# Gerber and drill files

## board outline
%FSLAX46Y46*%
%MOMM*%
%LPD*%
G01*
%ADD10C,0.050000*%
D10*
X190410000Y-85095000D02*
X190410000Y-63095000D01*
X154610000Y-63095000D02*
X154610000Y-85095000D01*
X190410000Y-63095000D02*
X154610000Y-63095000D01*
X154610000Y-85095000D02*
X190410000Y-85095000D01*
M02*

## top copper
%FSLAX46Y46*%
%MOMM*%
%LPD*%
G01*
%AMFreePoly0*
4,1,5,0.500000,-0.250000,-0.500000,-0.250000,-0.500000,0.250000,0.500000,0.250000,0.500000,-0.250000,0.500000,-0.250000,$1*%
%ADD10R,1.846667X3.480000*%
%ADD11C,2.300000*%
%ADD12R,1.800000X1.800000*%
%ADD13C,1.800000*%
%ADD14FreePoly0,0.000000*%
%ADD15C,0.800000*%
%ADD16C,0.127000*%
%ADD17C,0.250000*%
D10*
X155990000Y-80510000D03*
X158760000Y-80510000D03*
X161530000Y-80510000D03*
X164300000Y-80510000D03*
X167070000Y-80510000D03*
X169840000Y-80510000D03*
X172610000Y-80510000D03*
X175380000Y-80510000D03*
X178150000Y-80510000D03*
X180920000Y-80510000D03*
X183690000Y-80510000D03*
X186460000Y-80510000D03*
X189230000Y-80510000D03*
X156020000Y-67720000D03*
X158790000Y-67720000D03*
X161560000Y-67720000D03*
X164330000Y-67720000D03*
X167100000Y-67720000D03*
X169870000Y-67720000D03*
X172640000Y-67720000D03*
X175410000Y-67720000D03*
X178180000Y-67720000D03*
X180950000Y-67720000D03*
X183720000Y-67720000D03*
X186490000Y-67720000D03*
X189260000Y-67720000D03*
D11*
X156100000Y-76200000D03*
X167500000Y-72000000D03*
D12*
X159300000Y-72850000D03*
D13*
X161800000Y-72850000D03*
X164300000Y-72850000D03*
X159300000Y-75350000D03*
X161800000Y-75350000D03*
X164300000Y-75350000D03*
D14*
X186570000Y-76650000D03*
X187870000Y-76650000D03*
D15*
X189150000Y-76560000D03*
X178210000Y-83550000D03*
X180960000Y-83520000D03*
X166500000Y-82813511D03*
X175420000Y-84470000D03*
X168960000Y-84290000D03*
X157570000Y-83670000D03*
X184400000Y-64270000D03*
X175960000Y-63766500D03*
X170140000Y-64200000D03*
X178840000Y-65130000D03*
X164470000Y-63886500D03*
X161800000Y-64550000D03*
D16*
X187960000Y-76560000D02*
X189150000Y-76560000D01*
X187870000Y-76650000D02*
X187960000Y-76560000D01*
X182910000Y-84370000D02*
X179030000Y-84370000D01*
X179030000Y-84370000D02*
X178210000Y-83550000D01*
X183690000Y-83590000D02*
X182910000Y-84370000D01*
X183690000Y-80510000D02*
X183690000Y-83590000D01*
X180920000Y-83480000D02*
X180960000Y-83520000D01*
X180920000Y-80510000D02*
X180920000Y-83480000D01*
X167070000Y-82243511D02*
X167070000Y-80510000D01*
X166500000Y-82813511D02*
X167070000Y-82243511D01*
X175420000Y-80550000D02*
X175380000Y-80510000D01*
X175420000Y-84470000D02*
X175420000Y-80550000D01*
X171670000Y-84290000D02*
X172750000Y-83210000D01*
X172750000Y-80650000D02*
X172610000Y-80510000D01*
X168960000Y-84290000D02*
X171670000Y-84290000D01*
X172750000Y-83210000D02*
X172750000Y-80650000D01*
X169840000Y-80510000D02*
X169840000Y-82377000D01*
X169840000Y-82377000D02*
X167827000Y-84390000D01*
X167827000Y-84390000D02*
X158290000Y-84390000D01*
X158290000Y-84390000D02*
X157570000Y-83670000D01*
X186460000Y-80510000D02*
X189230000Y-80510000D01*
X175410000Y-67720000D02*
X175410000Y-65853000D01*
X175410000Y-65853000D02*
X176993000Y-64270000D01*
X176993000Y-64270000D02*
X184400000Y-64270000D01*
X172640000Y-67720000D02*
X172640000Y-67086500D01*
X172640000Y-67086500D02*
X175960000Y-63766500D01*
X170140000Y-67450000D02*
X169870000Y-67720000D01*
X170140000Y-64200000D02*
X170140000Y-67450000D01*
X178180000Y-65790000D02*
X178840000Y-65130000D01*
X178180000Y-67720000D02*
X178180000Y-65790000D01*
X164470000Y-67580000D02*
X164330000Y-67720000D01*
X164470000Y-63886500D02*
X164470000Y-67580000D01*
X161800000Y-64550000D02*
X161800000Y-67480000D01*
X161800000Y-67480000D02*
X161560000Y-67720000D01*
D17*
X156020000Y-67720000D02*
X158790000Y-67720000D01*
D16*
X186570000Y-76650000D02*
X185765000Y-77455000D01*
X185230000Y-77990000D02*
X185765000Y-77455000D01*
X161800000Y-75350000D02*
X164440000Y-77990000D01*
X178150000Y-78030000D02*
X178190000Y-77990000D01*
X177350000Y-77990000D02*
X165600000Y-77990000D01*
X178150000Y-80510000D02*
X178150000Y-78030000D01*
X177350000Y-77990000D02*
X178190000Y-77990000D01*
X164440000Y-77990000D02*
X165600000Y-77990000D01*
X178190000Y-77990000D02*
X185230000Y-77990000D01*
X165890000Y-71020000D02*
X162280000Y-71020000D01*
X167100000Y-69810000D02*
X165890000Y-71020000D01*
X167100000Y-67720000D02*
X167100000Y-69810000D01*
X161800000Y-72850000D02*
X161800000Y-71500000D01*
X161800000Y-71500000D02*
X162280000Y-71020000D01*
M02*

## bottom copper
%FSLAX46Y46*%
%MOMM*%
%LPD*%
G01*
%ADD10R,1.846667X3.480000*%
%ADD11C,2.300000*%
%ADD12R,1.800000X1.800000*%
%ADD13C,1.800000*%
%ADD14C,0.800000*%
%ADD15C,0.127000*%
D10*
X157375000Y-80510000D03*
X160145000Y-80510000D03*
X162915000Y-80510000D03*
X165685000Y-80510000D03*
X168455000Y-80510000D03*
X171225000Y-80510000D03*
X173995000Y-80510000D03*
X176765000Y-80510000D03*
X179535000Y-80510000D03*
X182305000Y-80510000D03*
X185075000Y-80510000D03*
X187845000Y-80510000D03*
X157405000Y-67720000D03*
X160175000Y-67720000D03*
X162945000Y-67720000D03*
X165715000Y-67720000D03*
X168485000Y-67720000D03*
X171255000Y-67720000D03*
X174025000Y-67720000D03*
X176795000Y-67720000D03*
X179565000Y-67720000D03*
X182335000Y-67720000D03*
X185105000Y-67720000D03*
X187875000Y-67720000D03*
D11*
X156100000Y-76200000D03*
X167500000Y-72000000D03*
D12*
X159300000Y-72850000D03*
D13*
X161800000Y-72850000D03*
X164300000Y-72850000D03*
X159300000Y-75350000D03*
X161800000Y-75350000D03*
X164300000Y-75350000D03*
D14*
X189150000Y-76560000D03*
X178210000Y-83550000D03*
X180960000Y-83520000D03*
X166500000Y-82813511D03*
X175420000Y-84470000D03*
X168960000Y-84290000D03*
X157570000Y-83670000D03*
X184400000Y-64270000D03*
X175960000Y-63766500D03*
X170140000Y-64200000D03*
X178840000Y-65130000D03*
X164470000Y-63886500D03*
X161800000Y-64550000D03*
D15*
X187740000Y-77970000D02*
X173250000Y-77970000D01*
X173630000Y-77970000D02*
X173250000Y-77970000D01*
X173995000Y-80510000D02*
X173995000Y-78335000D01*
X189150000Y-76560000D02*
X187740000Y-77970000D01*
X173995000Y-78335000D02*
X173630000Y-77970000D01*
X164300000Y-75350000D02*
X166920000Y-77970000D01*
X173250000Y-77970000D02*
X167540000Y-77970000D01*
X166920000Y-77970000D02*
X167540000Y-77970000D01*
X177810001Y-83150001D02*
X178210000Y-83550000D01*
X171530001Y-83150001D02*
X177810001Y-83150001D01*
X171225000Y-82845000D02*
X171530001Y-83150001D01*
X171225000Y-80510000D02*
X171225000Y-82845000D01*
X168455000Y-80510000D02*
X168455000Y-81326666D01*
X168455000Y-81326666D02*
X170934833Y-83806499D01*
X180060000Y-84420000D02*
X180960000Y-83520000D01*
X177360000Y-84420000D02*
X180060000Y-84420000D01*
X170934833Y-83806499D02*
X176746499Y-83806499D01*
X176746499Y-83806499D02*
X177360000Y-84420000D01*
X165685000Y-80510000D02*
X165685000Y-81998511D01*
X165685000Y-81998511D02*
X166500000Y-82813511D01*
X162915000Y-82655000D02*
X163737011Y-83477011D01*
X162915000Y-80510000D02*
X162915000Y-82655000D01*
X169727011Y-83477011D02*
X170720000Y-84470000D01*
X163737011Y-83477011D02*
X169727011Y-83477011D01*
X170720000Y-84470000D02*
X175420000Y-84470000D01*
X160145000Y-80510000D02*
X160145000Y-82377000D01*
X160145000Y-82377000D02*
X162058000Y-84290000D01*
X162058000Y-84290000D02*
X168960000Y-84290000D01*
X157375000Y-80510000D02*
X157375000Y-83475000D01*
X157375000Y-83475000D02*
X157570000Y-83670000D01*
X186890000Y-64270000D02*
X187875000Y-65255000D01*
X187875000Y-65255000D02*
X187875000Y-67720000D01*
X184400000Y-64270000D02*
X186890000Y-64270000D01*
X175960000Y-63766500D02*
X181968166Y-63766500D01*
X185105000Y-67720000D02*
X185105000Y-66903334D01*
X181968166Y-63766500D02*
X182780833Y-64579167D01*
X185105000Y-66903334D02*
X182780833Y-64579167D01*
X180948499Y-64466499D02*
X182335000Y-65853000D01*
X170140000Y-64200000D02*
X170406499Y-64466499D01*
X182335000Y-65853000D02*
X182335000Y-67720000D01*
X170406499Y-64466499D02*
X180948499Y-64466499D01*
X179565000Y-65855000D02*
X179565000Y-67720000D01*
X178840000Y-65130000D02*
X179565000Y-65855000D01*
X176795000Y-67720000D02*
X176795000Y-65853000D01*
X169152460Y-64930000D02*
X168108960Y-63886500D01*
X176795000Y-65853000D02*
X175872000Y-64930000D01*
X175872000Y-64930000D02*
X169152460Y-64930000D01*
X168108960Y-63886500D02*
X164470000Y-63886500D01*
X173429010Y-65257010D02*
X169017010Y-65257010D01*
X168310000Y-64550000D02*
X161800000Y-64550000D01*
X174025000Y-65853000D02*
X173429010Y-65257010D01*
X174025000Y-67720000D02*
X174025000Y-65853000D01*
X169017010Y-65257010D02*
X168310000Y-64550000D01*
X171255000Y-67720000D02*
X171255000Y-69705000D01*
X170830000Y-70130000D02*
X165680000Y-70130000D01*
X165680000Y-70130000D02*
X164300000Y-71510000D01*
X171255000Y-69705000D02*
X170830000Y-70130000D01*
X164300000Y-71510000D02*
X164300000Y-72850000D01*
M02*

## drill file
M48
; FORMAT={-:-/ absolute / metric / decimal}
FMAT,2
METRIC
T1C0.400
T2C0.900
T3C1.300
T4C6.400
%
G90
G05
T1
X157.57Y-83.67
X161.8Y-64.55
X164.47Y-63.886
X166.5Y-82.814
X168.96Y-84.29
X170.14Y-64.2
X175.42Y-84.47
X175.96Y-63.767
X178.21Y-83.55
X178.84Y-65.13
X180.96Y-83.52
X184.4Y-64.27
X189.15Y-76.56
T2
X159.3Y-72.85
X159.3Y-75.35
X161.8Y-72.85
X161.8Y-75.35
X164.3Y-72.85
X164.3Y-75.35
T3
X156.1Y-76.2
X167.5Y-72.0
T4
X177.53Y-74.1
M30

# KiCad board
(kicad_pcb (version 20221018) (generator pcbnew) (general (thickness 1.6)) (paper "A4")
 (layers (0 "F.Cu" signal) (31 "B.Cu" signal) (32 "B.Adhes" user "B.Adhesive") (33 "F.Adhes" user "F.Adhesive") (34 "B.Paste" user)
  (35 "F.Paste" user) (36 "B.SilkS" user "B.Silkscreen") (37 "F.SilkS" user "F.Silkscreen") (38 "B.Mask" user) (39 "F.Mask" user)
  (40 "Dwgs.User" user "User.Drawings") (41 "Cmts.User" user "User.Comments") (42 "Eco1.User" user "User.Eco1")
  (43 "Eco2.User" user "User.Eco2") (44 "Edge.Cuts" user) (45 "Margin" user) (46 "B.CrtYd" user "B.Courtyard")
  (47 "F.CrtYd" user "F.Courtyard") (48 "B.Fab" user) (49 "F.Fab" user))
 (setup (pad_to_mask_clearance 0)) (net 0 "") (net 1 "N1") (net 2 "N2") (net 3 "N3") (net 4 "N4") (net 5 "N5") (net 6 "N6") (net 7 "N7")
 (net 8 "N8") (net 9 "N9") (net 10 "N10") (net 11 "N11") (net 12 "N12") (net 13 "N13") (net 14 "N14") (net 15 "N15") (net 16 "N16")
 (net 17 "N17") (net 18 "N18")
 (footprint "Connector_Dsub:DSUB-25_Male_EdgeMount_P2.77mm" (layer "F.Cu") (at 172.61 80.51)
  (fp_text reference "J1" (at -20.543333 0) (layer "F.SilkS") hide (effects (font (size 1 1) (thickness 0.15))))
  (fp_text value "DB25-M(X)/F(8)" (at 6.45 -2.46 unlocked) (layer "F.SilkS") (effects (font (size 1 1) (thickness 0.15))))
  (pad "1" smd rect (at -16.62 0) (size 1.846667 3.48) (layers "F.Cu" "F.Paste" "F.Mask"))
  (pad "2" smd rect (at -13.85 0) (size 1.846667 3.48) (layers "F.Cu" "F.Paste" "F.Mask"))
  (pad "3" smd rect (at -11.08 0) (size 1.846667 3.48) (layers "F.Cu" "F.Paste" "F.Mask"))
  (pad "4" smd rect (at -8.31 0) (size 1.846667 3.48) (layers "F.Cu" "F.Paste" "F.Mask"))
  (pad "5" smd rect (at -5.54 0) (size 1.846667 3.48) (layers "F.Cu" "F.Paste" "F.Mask") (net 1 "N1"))
  (pad "6" smd rect (at -2.77 0) (size 1.846667 3.48) (layers "F.Cu" "F.Paste" "F.Mask") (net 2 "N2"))
  (pad "7" smd rect (at 0 0) (size 1.846667 3.48) (layers "F.Cu" "F.Paste" "F.Mask") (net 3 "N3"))
  (pad "8" smd rect (at 2.77 0) (size 1.846667 3.48) (layers "F.Cu" "F.Paste" "F.Mask") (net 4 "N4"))
  (pad "9" smd rect (at 5.54 0) (size 1.846667 3.48) (layers "F.Cu" "F.Paste" "F.Mask") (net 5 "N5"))
  (pad "10" smd rect (at 8.31 0) (size 1.846667 3.48) (layers "F.Cu" "F.Paste" "F.Mask") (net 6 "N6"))
  (pad "11" smd rect (at 11.08 0) (size 1.846667 3.48) (layers "F.Cu" "F.Paste" "F.Mask") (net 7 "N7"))
  (pad "12" smd rect (at 13.85 0) (size 1.846667 3.48) (layers "F.Cu" "F.Paste" "F.Mask") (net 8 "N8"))
  (pad "13" smd rect (at 16.62 0) (size 1.846667 3.48) (layers "F.Cu" "F.Paste" "F.Mask") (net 8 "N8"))
  (pad "14" smd rect (at -15.235 0) (size 1.846667 3.48) (layers "B.Cu" "B.Paste" "B.Mask") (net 2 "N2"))
  (pad "15" smd rect (at -12.465 0) (size 1.846667 3.48) (layers "B.Cu" "B.Paste" "B.Mask") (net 3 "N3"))
  (pad "16" smd rect (at -9.695 0) (size 1.846667 3.48) (layers "B.Cu" "B.Paste" "B.Mask") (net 4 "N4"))
  (pad "17" smd rect (at -6.925 0) (size 1.846667 3.48) (layers "B.Cu" "B.Paste" "B.Mask") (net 1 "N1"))
  (pad "18" smd rect (at -4.155 0) (size 1.846667 3.48) (layers "B.Cu" "B.Paste" "B.Mask") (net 6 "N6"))
  (pad "19" smd rect (at -1.385 0) (size 1.846667 3.48) (layers "B.Cu" "B.Paste" "B.Mask") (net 7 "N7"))
  (pad "20" smd rect (at 1.385 0) (size 1.846667 3.48) (layers "B.Cu" "B.Paste" "B.Mask") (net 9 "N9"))
  (pad "21" smd rect (at 4.155 0) (size 1.846667 3.48) (layers "B.Cu" "B.Paste" "B.Mask"))
  (pad "22" smd rect (at 6.925 0) (size 1.846667 3.48) (layers "B.Cu" "B.Paste" "B.Mask"))
  (pad "23" smd rect (at 9.695 0) (size 1.846667 3.48) (layers "B.Cu" "B.Paste" "B.Mask"))
  (pad "24" smd rect (at 12.465 0) (size 1.846667 3.48) (layers "B.Cu" "B.Paste" "B.Mask"))
  (pad "25" smd rect (at 15.235 0) (size 1.846667 3.48) (layers "B.Cu" "B.Paste" "B.Mask")))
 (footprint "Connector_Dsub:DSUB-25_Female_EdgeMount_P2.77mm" (layer "F.Cu") (at 172.64 67.72 180)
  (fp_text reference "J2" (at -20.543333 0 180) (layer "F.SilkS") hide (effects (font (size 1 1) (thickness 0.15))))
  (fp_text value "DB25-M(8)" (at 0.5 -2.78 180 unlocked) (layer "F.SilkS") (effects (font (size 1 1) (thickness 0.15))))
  (pad "1" smd rect (at 16.62 0 180) (size 1.846667 3.48) (layers "F.Cu" "F.Paste" "F.Mask") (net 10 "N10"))
  (pad "2" smd rect (at 13.85 0 180) (size 1.846667 3.48) (layers "F.Cu" "F.Paste" "F.Mask") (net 10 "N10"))
  (pad "3" smd rect (at 11.08 0 180) (size 1.846667 3.48) (layers "F.Cu" "F.Paste" "F.Mask") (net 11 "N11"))
  (pad "4" smd rect (at 8.31 0 180) (size 1.846667 3.48) (layers "F.Cu" "F.Paste" "F.Mask") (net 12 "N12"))
  (pad "5" smd rect (at 5.54 0 180) (size 1.846667 3.48) (layers "F.Cu" "F.Paste" "F.Mask") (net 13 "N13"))
  (pad "6" smd rect (at 2.77 0 180) (size 1.846667 3.48) (layers "F.Cu" "F.Paste" "F.Mask") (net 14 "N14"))
  (pad "7" smd rect (at 0 0 180) (size 1.846667 3.48) (layers "F.Cu" "F.Paste" "F.Mask") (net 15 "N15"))
  (pad "8" smd rect (at -2.77 0 180) (size 1.846667 3.48) (layers "F.Cu" "F.Paste" "F.Mask") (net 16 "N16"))
  (pad "9" smd rect (at -5.54 0 180) (size 1.846667 3.48) (layers "F.Cu" "F.Paste" "F.Mask") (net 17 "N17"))
  (pad "10" smd rect (at -8.31 0 180) (size 1.846667 3.48) (layers "F.Cu" "F.Paste" "F.Mask"))
  (pad "11" smd rect (at -11.08 0 180) (size 1.846667 3.48) (layers "F.Cu" "F.Paste" "F.Mask"))
  (pad "12" smd rect (at -13.85 0 180) (size 1.846667 3.48) (layers "F.Cu" "F.Paste" "F.Mask"))
  (pad "13" smd rect (at -16.62 0 180) (size 1.846667 3.48) (layers "F.Cu" "F.Paste" "F.Mask"))
  (pad "14" smd rect (at 15.235 0 180) (size 1.846667 3.48) (layers "B.Cu" "B.Paste" "B.Mask"))
  (pad "15" smd rect (at 12.465 0 180) (size 1.846667 3.48) (layers "B.Cu" "B.Paste" "B.Mask"))
  (pad "16" smd rect (at 9.695 0 180) (size 1.846667 3.48) (layers "B.Cu" "B.Paste" "B.Mask"))
  (pad "17" smd rect (at 6.925 0 180) (size 1.846667 3.48) (layers "B.Cu" "B.Paste" "B.Mask"))
  (pad "18" smd rect (at 4.155 0 180) (size 1.846667 3.48) (layers "B.Cu" "B.Paste" "B.Mask"))
  (pad "19" smd rect (at 1.385 0 180) (size 1.846667 3.48) (layers "B.Cu" "B.Paste" "B.Mask") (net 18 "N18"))
  (pad "20" smd rect (at -1.385 0 180) (size 1.846667 3.48) (layers "B.Cu" "B.Paste" "B.Mask") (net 11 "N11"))
  (pad "21" smd rect (at -4.155 0 180) (size 1.846667 3.48) (layers "B.Cu" "B.Paste" "B.Mask") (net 12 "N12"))
  (pad "22" smd rect (at -6.925 0 180) (size 1.846667 3.48) (layers "B.Cu" "B.Paste" "B.Mask") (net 17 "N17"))
  (pad "23" smd rect (at -9.695 0 180) (size 1.846667 3.48) (layers "B.Cu" "B.Paste" "B.Mask") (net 14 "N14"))
  (pad "24" smd rect (at -12.465 0 180) (size 1.846667 3.48) (layers "B.Cu" "B.Paste" "B.Mask") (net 15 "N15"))
  (pad "25" smd rect (at -15.235 0 180) (size 1.846667 3.48) (layers "B.Cu" "B.Paste" "B.Mask") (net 16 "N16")))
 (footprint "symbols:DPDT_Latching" (layer "F.Cu") (at 159.3 72.85)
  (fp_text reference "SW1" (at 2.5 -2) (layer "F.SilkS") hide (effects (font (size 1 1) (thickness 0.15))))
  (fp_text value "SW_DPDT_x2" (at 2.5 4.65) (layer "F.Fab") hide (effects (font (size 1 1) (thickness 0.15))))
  (pad "" thru_hole circle (at -3.2 3.35) (size 2.3 2.3) (drill 1.3) (layers "*.Cu" "B.Mask"))
  (pad "" thru_hole circle (at 8.2 -0.85) (size 2.3 2.3) (drill 1.3) (layers "*.Cu" "B.Mask"))
  (pad "1" thru_hole rect (at 0 0) (size 1.8 1.8) (drill 0.9) (layers "*.Cu" "B.Mask"))
  (pad "2" thru_hole circle (at 2.5 0) (size 1.8 1.8) (drill 0.9) (layers "*.Cu" "B.Mask") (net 13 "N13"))
  (pad "3" thru_hole circle (at 5 0) (size 1.8 1.8) (drill 0.9) (layers "*.Cu" "B.Mask") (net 18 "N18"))
  (pad "4" thru_hole circle (at 0 2.5) (size 1.8 1.8) (drill 0.9) (layers "*.Cu" "B.Mask"))
  (pad "5" thru_hole circle (at 2.5 2.5) (size 1.8 1.8) (drill 0.9) (layers "*.Cu" "B.Mask") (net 5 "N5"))
  (pad "6" thru_hole circle (at 5 2.5) (size 1.8 1.8) (drill 0.9) (layers "*.Cu" "B.Mask") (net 9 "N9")))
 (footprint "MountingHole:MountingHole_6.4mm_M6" (layer "F.Cu") (at 177.53 74.1)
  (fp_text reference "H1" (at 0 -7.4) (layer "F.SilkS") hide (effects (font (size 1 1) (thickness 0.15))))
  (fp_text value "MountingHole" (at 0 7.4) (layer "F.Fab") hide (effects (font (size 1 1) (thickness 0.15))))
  (pad "" np_thru_hole circle (at 0 0) (size 6.4 6.4) (drill 6.4) (layers "*.Cu" "*.Mask")))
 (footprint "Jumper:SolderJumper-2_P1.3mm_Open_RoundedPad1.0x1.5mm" (layer "F.Cu") (at 187.22 76.65)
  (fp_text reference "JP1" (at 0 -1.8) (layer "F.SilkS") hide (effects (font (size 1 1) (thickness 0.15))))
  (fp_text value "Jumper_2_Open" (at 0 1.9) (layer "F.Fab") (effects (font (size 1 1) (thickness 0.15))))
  (pad "1" smd custom (at -0.65 0) (size 1 0.5) (layers "F.Cu" "F.Mask") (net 5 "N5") (zone_connect 2)
   (options (clearance outline) (anchor rect)) (primitives))
  (pad "2" smd custom (at 0.65 0) (size 1 0.5) (layers "F.Cu" "F.Mask") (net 9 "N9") (zone_connect 2)
   (options (clearance outline) (anchor rect)) (primitives)))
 (gr_line (start 190.41 85.095) (end 190.41 63.095) (stroke (width 0.05) (type solid)) (layer "Edge.Cuts"))
 (gr_line (start 154.61 63.095) (end 154.61 85.095) (stroke (width 0.05) (type solid)) (layer "Edge.Cuts"))
 (gr_line (start 190.41 63.095) (end 154.61 63.095) (stroke (width 0.05) (type solid)) (layer "Edge.Cuts"))
 (gr_line (start 154.61 85.095) (end 190.41 85.095) (stroke (width 0.05) (type solid)) (layer "Edge.Cuts"))
 (segment (start 187.96 76.56) (end 189.15 76.56) (width 0.127) (layer "F.Cu") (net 9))
 (segment (start 187.87 76.65) (end 187.96 76.56) (width 0.127) (layer "F.Cu") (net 9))
 (via (at 189.15 76.56) (size 0.8) (drill 0.4) (layers "F.Cu" "B.Cu") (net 9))
 (segment (start 187.74 77.97) (end 173.25 77.97) (width 0.127) (layer "B.Cu") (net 9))
 (segment (start 173.63 77.97) (end 173.25 77.97) (width 0.127) (layer "B.Cu") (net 9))
 (segment (start 173.995 80.51) (end 173.995 78.335) (width 0.127) (layer "B.Cu") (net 9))
 (segment (start 189.15 76.56) (end 187.74 77.97) (width 0.127) (layer "B.Cu") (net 9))
 (segment (start 173.995 78.335) (end 173.63 77.97) (width 0.127) (layer "B.Cu") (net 9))
 (segment (start 164.3 75.35) (end 166.92 77.97) (width 0.127) (layer "B.Cu") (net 9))
 (segment (start 173.25 77.97) (end 167.54 77.97) (width 0.127) (layer "B.Cu") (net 9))
 (segment (start 166.92 77.97) (end 167.54 77.97) (width 0.127) (layer "B.Cu") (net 9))
 (segment (start 182.91 84.37) (end 179.03 84.37) (width 0.127) (layer "F.Cu") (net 7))
 (segment (start 179.03 84.37) (end 178.21 83.55) (width 0.127) (layer "F.Cu") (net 7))
 (segment (start 183.69 83.59) (end 182.91 84.37) (width 0.127) (layer "F.Cu") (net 7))
 (segment (start 183.69 80.51) (end 183.69 83.59) (width 0.127) (layer "F.Cu") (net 7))
 (via (at 178.21 83.55) (size 0.8) (drill 0.4) (layers "F.Cu" "B.Cu") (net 7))
 (segment (start 177.810001 83.150001) (end 178.21 83.55) (width 0.127) (layer "B.Cu") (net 7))
 (segment (start 171.530001 83.150001) (end 177.810001 83.150001) (width 0.127) (layer "B.Cu") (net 7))
 (segment (start 171.225 82.845) (end 171.530001 83.150001) (width 0.127) (layer "B.Cu") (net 7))
 (segment (start 171.225 80.51) (end 171.225 82.845) (width 0.127) (layer "B.Cu") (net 7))
 (segment (start 180.92 83.48) (end 180.96 83.52) (width 0.127) (layer "F.Cu") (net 6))
 (segment (start 180.92 80.51) (end 180.92 83.48) (width 0.127) (layer "F.Cu") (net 6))
 (via (at 180.96 83.52) (size 0.8) (drill 0.4) (layers "F.Cu" "B.Cu") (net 6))
 (segment (start 168.455 80.51) (end 168.455 81.326666) (width 0.127) (layer "B.Cu") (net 6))
 (segment (start 168.455 81.326666) (end 170.934833 83.806499) (width 0.127) (layer "B.Cu") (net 6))
 (segment (start 180.06 84.42) (end 180.96 83.52) (width 0.127) (layer "B.Cu") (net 6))
 (segment (start 177.36 84.42) (end 180.06 84.42) (width 0.127) (layer "B.Cu") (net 6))
 (segment (start 170.934833 83.806499) (end 176.746499 83.806499) (width 0.127) (layer "B.Cu") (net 6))
 (segment (start 176.746499 83.806499) (end 177.36 84.42) (width 0.127) (layer "B.Cu") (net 6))
 (segment (start 167.07 82.243511) (end 167.07 80.51) (width 0.127) (layer "F.Cu") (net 1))
 (segment (start 166.5 82.813511) (end 167.07 82.243511) (width 0.127) (layer "F.Cu") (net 1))
 (via (at 166.5 82.813511) (size 0.8) (drill 0.4) (layers "F.Cu" "B.Cu") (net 1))
 (segment (start 165.685 80.51) (end 165.685 81.998511) (width 0.127) (layer "B.Cu") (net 1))
 (segment (start 165.685 81.998511) (end 166.5 82.813511) (width 0.127) (layer "B.Cu") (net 1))
 (segment (start 175.42 80.55) (end 175.38 80.51) (width 0.127) (layer "F.Cu") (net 4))
 (segment (start 175.42 84.47) (end 175.42 80.55) (width 0.127) (layer "F.Cu") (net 4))
 (via (at 175.42 84.47) (size 0.8) (drill 0.4) (layers "F.Cu" "B.Cu") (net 4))
 (segment (start 162.915 82.655) (end 163.737011 83.477011) (width 0.127) (layer "B.Cu") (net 4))
 (segment (start 162.915 80.51) (end 162.915 82.655) (width 0.127) (layer "B.Cu") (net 4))
 (segment (start 169.727011 83.477011) (end 170.72 84.47) (width 0.127) (layer "B.Cu") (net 4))
 (segment (start 163.737011 83.477011) (end 169.727011 83.477011) (width 0.127) (layer "B.Cu") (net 4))
 (segment (start 170.72 84.47) (end 175.42 84.47) (width 0.127) (layer "B.Cu") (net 4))
 (segment (start 171.67 84.29) (end 172.75 83.21) (width 0.127) (layer "F.Cu") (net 3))
 (segment (start 172.75 80.65) (end 172.61 80.51) (width 0.127) (layer "F.Cu") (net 3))
 (segment (start 168.96 84.29) (end 171.67 84.29) (width 0.127) (layer "F.Cu") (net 3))
 (segment (start 172.75 83.21) (end 172.75 80.65) (width 0.127) (layer "F.Cu") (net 3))
 (via (at 168.96 84.29) (size 0.8) (drill 0.4) (layers "F.Cu" "B.Cu") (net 3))
 (segment (start 160.145 80.51) (end 160.145 82.377) (width 0.127) (layer "B.Cu") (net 3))
 (segment (start 160.145 82.377) (end 162.058 84.29) (width 0.127) (layer "B.Cu") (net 3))
 (segment (start 162.058 84.29) (end 168.96 84.29) (width 0.127) (layer "B.Cu") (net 3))
 (segment (start 169.84 80.51) (end 169.84 82.377) (width 0.127) (layer "F.Cu") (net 2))
 (segment (start 169.84 82.377) (end 167.827 84.39) (width 0.127) (layer "F.Cu") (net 2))
 (segment (start 167.827 84.39) (end 158.29 84.39) (width 0.127) (layer "F.Cu") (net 2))
 (segment (start 158.29 84.39) (end 157.57 83.67) (width 0.127) (layer "F.Cu") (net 2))
 (via (at 157.57 83.67) (size 0.8) (drill 0.4) (layers "F.Cu" "B.Cu") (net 2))
 (segment (start 157.375 80.51) (end 157.375 83.475) (width 0.127) (layer "B.Cu") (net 2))
 (segment (start 157.375 83.475) (end 157.57 83.67) (width 0.127) (layer "B.Cu") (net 2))
 (segment (start 186.46 80.51) (end 189.23 80.51) (width 0.127) (layer "F.Cu") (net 8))
 (segment (start 175.41 67.72) (end 175.41 65.853) (width 0.127) (layer "F.Cu") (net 16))
 (segment (start 175.41 65.853) (end 176.993 64.27) (width 0.127) (layer "F.Cu") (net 16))
 (segment (start 176.993 64.27) (end 184.4 64.27) (width 0.127) (layer "F.Cu") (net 16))
 (via (at 184.4 64.27) (size 0.8) (drill 0.4) (layers "F.Cu" "B.Cu") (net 16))
 (segment (start 186.89 64.27) (end 187.875 65.255) (width 0.127) (layer "B.Cu") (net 16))
 (segment (start 187.875 65.255) (end 187.875 67.72) (width 0.127) (layer "B.Cu") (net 16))
 (segment (start 184.4 64.27) (end 186.89 64.27) (width 0.127) (layer "B.Cu") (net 16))
 (segment (start 172.64 67.72) (end 172.64 67.0865) (width 0.127) (layer "F.Cu") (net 15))
 (segment (start 172.64 67.0865) (end 175.96 63.7665) (width 0.127) (layer "F.Cu") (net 15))
 (via (at 175.96 63.7665) (size 0.8) (drill 0.4) (layers "F.Cu" "B.Cu") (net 15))
 (segment (start 175.96 63.7665) (end 181.968166 63.7665) (width 0.127) (layer "B.Cu") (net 15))
 (segment (start 185.105 67.72) (end 185.105 66.903334) (width 0.127) (layer "B.Cu") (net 15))
 (segment (start 181.968166 63.7665) (end 182.780833 64.579167) (width 0.127) (layer "B.Cu") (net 15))
 (segment (start 185.105 66.903334) (end 182.780833 64.579167) (width 0.127) (layer "B.Cu") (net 15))
 (segment (start 170.14 67.45) (end 169.87 67.72) (width 0.127) (layer "F.Cu") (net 14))
 (segment (start 170.14 64.2) (end 170.14 67.45) (width 0.127) (layer "F.Cu") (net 14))
 (via (at 170.14 64.2) (size 0.8) (drill 0.4) (layers "F.Cu" "B.Cu") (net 14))
 (segment (start 180.948499 64.466499) (end 182.335 65.853) (width 0.127) (layer "B.Cu") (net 14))
 (segment (start 170.14 64.2) (end 170.406499 64.466499) (width 0.127) (layer "B.Cu") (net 14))
 (segment (start 182.335 65.853) (end 182.335 67.72) (width 0.127) (layer "B.Cu") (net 14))
 (segment (start 170.406499 64.466499) (end 180.948499 64.466499) (width 0.127) (layer "B.Cu") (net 14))
 (segment (start 178.18 65.79) (end 178.84 65.13) (width 0.127) (layer "F.Cu") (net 17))
 (segment (start 178.18 67.72) (end 178.18 65.79) (width 0.127) (layer "F.Cu") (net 17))
 (via (at 178.84 65.13) (size 0.8) (drill 0.4) (layers "F.Cu" "B.Cu") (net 17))
 (segment (start 179.565 65.855) (end 179.565 67.72) (width 0.127) (layer "B.Cu") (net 17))
 (segment (start 178.84 65.13) (end 179.565 65.855) (width 0.127) (layer "B.Cu") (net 17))
 (segment (start 164.47 67.58) (end 164.33 67.72) (width 0.127) (layer "F.Cu") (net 12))
 (segment (start 164.47 63.8865) (end 164.47 67.58) (width 0.127) (layer "F.Cu") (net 12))
 (via (at 164.47 63.8865) (size 0.8) (drill 0.4) (layers "F.Cu" "B.Cu") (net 12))
 (segment (start 176.795 67.72) (end 176.795 65.853) (width 0.127) (layer "B.Cu") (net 12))
 (segment (start 169.15246 64.93) (end 168.10896 63.8865) (width 0.127) (layer "B.Cu") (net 12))
 (segment (start 176.795 65.853) (end 175.872 64.93) (width 0.127) (layer "B.Cu") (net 12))
 (segment (start 175.872 64.93) (end 169.15246 64.93) (width 0.127) (layer "B.Cu") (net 12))
 (segment (start 168.10896 63.8865) (end 164.47 63.8865) (width 0.127) (layer "B.Cu") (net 12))
 (segment (start 161.8 64.55) (end 161.8 67.48) (width 0.127) (layer "F.Cu") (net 11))
 (segment (start 161.8 67.48) (end 161.56 67.72) (width 0.127) (layer "F.Cu") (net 11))
 (via (at 161.8 64.55) (size 0.8) (drill 0.4) (layers "F.Cu" "B.Cu") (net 11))
 (segment (start 173.42901 65.25701) (end 169.01701 65.25701) (width 0.127) (layer "B.Cu") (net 11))
 (segment (start 168.31 64.55) (end 161.8 64.55) (width 0.127) (layer "B.Cu") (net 11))
 (segment (start 174.025 65.853) (end 173.42901 65.25701) (width 0.127) (layer "B.Cu") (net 11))
 (segment (start 174.025 67.72) (end 174.025 65.853) (width 0.127) (layer "B.Cu") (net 11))
 (segment (start 169.01701 65.25701) (end 168.31 64.55) (width 0.127) (layer "B.Cu") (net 11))
 (segment (start 171.255 67.72) (end 171.255 69.705) (width 0.127) (layer "B.Cu") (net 18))
 (segment (start 170.83 70.13) (end 165.68 70.13) (width 0.127) (layer "B.Cu") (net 18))
 (segment (start 165.68 70.13) (end 164.3 71.51) (width 0.127) (layer "B.Cu") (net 18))
 (segment (start 171.255 69.705) (end 170.83 70.13) (width 0.127) (layer "B.Cu") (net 18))
 (segment (start 164.3 71.51) (end 164.3 72.85) (width 0.127) (layer "B.Cu") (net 18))
 (segment (start 156.02 67.72) (end 158.79 67.72) (width 0.25) (layer "F.Cu") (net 10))
 (segment (start 186.57 76.65) (end 185.765 77.455) (width 0.127) (layer "F.Cu") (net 5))
 (segment (start 185.23 77.99) (end 185.765 77.455) (width 0.127) (layer "F.Cu") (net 5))
 (segment (start 161.8 75.35) (end 164.44 77.99) (width 0.127) (layer "F.Cu") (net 5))
 (segment (start 178.15 78.03) (end 178.19 77.99) (width 0.127) (layer "F.Cu") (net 5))
 (segment (start 177.35 77.99) (end 165.6 77.99) (width 0.127) (layer "F.Cu") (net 5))
 (segment (start 178.15 80.51) (end 178.15 78.03) (width 0.127) (layer "F.Cu") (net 5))
 (segment (start 177.35 77.99) (end 178.19 77.99) (width 0.127) (layer "F.Cu") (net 5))
 (segment (start 164.44 77.99) (end 165.6 77.99) (width 0.127) (layer "F.Cu") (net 5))
 (segment (start 178.19 77.99) (end 185.23 77.99) (width 0.127) (layer "F.Cu") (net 5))
 (segment (start 165.89 71.02) (end 162.28 71.02) (width 0.127) (layer "F.Cu") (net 13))
 (segment (start 167.1 69.81) (end 165.89 71.02) (width 0.127) (layer "F.Cu") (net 13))
 (segment (start 167.1 67.72) (end 167.1 69.81) (width 0.127) (layer "F.Cu") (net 13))
 (segment (start 161.8 72.85) (end 161.8 71.5) (width 0.127) (layer "F.Cu") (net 13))
 (segment (start 161.8 71.5) (end 162.28 71.02) (width 0.127) (layer "F.Cu") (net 13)))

